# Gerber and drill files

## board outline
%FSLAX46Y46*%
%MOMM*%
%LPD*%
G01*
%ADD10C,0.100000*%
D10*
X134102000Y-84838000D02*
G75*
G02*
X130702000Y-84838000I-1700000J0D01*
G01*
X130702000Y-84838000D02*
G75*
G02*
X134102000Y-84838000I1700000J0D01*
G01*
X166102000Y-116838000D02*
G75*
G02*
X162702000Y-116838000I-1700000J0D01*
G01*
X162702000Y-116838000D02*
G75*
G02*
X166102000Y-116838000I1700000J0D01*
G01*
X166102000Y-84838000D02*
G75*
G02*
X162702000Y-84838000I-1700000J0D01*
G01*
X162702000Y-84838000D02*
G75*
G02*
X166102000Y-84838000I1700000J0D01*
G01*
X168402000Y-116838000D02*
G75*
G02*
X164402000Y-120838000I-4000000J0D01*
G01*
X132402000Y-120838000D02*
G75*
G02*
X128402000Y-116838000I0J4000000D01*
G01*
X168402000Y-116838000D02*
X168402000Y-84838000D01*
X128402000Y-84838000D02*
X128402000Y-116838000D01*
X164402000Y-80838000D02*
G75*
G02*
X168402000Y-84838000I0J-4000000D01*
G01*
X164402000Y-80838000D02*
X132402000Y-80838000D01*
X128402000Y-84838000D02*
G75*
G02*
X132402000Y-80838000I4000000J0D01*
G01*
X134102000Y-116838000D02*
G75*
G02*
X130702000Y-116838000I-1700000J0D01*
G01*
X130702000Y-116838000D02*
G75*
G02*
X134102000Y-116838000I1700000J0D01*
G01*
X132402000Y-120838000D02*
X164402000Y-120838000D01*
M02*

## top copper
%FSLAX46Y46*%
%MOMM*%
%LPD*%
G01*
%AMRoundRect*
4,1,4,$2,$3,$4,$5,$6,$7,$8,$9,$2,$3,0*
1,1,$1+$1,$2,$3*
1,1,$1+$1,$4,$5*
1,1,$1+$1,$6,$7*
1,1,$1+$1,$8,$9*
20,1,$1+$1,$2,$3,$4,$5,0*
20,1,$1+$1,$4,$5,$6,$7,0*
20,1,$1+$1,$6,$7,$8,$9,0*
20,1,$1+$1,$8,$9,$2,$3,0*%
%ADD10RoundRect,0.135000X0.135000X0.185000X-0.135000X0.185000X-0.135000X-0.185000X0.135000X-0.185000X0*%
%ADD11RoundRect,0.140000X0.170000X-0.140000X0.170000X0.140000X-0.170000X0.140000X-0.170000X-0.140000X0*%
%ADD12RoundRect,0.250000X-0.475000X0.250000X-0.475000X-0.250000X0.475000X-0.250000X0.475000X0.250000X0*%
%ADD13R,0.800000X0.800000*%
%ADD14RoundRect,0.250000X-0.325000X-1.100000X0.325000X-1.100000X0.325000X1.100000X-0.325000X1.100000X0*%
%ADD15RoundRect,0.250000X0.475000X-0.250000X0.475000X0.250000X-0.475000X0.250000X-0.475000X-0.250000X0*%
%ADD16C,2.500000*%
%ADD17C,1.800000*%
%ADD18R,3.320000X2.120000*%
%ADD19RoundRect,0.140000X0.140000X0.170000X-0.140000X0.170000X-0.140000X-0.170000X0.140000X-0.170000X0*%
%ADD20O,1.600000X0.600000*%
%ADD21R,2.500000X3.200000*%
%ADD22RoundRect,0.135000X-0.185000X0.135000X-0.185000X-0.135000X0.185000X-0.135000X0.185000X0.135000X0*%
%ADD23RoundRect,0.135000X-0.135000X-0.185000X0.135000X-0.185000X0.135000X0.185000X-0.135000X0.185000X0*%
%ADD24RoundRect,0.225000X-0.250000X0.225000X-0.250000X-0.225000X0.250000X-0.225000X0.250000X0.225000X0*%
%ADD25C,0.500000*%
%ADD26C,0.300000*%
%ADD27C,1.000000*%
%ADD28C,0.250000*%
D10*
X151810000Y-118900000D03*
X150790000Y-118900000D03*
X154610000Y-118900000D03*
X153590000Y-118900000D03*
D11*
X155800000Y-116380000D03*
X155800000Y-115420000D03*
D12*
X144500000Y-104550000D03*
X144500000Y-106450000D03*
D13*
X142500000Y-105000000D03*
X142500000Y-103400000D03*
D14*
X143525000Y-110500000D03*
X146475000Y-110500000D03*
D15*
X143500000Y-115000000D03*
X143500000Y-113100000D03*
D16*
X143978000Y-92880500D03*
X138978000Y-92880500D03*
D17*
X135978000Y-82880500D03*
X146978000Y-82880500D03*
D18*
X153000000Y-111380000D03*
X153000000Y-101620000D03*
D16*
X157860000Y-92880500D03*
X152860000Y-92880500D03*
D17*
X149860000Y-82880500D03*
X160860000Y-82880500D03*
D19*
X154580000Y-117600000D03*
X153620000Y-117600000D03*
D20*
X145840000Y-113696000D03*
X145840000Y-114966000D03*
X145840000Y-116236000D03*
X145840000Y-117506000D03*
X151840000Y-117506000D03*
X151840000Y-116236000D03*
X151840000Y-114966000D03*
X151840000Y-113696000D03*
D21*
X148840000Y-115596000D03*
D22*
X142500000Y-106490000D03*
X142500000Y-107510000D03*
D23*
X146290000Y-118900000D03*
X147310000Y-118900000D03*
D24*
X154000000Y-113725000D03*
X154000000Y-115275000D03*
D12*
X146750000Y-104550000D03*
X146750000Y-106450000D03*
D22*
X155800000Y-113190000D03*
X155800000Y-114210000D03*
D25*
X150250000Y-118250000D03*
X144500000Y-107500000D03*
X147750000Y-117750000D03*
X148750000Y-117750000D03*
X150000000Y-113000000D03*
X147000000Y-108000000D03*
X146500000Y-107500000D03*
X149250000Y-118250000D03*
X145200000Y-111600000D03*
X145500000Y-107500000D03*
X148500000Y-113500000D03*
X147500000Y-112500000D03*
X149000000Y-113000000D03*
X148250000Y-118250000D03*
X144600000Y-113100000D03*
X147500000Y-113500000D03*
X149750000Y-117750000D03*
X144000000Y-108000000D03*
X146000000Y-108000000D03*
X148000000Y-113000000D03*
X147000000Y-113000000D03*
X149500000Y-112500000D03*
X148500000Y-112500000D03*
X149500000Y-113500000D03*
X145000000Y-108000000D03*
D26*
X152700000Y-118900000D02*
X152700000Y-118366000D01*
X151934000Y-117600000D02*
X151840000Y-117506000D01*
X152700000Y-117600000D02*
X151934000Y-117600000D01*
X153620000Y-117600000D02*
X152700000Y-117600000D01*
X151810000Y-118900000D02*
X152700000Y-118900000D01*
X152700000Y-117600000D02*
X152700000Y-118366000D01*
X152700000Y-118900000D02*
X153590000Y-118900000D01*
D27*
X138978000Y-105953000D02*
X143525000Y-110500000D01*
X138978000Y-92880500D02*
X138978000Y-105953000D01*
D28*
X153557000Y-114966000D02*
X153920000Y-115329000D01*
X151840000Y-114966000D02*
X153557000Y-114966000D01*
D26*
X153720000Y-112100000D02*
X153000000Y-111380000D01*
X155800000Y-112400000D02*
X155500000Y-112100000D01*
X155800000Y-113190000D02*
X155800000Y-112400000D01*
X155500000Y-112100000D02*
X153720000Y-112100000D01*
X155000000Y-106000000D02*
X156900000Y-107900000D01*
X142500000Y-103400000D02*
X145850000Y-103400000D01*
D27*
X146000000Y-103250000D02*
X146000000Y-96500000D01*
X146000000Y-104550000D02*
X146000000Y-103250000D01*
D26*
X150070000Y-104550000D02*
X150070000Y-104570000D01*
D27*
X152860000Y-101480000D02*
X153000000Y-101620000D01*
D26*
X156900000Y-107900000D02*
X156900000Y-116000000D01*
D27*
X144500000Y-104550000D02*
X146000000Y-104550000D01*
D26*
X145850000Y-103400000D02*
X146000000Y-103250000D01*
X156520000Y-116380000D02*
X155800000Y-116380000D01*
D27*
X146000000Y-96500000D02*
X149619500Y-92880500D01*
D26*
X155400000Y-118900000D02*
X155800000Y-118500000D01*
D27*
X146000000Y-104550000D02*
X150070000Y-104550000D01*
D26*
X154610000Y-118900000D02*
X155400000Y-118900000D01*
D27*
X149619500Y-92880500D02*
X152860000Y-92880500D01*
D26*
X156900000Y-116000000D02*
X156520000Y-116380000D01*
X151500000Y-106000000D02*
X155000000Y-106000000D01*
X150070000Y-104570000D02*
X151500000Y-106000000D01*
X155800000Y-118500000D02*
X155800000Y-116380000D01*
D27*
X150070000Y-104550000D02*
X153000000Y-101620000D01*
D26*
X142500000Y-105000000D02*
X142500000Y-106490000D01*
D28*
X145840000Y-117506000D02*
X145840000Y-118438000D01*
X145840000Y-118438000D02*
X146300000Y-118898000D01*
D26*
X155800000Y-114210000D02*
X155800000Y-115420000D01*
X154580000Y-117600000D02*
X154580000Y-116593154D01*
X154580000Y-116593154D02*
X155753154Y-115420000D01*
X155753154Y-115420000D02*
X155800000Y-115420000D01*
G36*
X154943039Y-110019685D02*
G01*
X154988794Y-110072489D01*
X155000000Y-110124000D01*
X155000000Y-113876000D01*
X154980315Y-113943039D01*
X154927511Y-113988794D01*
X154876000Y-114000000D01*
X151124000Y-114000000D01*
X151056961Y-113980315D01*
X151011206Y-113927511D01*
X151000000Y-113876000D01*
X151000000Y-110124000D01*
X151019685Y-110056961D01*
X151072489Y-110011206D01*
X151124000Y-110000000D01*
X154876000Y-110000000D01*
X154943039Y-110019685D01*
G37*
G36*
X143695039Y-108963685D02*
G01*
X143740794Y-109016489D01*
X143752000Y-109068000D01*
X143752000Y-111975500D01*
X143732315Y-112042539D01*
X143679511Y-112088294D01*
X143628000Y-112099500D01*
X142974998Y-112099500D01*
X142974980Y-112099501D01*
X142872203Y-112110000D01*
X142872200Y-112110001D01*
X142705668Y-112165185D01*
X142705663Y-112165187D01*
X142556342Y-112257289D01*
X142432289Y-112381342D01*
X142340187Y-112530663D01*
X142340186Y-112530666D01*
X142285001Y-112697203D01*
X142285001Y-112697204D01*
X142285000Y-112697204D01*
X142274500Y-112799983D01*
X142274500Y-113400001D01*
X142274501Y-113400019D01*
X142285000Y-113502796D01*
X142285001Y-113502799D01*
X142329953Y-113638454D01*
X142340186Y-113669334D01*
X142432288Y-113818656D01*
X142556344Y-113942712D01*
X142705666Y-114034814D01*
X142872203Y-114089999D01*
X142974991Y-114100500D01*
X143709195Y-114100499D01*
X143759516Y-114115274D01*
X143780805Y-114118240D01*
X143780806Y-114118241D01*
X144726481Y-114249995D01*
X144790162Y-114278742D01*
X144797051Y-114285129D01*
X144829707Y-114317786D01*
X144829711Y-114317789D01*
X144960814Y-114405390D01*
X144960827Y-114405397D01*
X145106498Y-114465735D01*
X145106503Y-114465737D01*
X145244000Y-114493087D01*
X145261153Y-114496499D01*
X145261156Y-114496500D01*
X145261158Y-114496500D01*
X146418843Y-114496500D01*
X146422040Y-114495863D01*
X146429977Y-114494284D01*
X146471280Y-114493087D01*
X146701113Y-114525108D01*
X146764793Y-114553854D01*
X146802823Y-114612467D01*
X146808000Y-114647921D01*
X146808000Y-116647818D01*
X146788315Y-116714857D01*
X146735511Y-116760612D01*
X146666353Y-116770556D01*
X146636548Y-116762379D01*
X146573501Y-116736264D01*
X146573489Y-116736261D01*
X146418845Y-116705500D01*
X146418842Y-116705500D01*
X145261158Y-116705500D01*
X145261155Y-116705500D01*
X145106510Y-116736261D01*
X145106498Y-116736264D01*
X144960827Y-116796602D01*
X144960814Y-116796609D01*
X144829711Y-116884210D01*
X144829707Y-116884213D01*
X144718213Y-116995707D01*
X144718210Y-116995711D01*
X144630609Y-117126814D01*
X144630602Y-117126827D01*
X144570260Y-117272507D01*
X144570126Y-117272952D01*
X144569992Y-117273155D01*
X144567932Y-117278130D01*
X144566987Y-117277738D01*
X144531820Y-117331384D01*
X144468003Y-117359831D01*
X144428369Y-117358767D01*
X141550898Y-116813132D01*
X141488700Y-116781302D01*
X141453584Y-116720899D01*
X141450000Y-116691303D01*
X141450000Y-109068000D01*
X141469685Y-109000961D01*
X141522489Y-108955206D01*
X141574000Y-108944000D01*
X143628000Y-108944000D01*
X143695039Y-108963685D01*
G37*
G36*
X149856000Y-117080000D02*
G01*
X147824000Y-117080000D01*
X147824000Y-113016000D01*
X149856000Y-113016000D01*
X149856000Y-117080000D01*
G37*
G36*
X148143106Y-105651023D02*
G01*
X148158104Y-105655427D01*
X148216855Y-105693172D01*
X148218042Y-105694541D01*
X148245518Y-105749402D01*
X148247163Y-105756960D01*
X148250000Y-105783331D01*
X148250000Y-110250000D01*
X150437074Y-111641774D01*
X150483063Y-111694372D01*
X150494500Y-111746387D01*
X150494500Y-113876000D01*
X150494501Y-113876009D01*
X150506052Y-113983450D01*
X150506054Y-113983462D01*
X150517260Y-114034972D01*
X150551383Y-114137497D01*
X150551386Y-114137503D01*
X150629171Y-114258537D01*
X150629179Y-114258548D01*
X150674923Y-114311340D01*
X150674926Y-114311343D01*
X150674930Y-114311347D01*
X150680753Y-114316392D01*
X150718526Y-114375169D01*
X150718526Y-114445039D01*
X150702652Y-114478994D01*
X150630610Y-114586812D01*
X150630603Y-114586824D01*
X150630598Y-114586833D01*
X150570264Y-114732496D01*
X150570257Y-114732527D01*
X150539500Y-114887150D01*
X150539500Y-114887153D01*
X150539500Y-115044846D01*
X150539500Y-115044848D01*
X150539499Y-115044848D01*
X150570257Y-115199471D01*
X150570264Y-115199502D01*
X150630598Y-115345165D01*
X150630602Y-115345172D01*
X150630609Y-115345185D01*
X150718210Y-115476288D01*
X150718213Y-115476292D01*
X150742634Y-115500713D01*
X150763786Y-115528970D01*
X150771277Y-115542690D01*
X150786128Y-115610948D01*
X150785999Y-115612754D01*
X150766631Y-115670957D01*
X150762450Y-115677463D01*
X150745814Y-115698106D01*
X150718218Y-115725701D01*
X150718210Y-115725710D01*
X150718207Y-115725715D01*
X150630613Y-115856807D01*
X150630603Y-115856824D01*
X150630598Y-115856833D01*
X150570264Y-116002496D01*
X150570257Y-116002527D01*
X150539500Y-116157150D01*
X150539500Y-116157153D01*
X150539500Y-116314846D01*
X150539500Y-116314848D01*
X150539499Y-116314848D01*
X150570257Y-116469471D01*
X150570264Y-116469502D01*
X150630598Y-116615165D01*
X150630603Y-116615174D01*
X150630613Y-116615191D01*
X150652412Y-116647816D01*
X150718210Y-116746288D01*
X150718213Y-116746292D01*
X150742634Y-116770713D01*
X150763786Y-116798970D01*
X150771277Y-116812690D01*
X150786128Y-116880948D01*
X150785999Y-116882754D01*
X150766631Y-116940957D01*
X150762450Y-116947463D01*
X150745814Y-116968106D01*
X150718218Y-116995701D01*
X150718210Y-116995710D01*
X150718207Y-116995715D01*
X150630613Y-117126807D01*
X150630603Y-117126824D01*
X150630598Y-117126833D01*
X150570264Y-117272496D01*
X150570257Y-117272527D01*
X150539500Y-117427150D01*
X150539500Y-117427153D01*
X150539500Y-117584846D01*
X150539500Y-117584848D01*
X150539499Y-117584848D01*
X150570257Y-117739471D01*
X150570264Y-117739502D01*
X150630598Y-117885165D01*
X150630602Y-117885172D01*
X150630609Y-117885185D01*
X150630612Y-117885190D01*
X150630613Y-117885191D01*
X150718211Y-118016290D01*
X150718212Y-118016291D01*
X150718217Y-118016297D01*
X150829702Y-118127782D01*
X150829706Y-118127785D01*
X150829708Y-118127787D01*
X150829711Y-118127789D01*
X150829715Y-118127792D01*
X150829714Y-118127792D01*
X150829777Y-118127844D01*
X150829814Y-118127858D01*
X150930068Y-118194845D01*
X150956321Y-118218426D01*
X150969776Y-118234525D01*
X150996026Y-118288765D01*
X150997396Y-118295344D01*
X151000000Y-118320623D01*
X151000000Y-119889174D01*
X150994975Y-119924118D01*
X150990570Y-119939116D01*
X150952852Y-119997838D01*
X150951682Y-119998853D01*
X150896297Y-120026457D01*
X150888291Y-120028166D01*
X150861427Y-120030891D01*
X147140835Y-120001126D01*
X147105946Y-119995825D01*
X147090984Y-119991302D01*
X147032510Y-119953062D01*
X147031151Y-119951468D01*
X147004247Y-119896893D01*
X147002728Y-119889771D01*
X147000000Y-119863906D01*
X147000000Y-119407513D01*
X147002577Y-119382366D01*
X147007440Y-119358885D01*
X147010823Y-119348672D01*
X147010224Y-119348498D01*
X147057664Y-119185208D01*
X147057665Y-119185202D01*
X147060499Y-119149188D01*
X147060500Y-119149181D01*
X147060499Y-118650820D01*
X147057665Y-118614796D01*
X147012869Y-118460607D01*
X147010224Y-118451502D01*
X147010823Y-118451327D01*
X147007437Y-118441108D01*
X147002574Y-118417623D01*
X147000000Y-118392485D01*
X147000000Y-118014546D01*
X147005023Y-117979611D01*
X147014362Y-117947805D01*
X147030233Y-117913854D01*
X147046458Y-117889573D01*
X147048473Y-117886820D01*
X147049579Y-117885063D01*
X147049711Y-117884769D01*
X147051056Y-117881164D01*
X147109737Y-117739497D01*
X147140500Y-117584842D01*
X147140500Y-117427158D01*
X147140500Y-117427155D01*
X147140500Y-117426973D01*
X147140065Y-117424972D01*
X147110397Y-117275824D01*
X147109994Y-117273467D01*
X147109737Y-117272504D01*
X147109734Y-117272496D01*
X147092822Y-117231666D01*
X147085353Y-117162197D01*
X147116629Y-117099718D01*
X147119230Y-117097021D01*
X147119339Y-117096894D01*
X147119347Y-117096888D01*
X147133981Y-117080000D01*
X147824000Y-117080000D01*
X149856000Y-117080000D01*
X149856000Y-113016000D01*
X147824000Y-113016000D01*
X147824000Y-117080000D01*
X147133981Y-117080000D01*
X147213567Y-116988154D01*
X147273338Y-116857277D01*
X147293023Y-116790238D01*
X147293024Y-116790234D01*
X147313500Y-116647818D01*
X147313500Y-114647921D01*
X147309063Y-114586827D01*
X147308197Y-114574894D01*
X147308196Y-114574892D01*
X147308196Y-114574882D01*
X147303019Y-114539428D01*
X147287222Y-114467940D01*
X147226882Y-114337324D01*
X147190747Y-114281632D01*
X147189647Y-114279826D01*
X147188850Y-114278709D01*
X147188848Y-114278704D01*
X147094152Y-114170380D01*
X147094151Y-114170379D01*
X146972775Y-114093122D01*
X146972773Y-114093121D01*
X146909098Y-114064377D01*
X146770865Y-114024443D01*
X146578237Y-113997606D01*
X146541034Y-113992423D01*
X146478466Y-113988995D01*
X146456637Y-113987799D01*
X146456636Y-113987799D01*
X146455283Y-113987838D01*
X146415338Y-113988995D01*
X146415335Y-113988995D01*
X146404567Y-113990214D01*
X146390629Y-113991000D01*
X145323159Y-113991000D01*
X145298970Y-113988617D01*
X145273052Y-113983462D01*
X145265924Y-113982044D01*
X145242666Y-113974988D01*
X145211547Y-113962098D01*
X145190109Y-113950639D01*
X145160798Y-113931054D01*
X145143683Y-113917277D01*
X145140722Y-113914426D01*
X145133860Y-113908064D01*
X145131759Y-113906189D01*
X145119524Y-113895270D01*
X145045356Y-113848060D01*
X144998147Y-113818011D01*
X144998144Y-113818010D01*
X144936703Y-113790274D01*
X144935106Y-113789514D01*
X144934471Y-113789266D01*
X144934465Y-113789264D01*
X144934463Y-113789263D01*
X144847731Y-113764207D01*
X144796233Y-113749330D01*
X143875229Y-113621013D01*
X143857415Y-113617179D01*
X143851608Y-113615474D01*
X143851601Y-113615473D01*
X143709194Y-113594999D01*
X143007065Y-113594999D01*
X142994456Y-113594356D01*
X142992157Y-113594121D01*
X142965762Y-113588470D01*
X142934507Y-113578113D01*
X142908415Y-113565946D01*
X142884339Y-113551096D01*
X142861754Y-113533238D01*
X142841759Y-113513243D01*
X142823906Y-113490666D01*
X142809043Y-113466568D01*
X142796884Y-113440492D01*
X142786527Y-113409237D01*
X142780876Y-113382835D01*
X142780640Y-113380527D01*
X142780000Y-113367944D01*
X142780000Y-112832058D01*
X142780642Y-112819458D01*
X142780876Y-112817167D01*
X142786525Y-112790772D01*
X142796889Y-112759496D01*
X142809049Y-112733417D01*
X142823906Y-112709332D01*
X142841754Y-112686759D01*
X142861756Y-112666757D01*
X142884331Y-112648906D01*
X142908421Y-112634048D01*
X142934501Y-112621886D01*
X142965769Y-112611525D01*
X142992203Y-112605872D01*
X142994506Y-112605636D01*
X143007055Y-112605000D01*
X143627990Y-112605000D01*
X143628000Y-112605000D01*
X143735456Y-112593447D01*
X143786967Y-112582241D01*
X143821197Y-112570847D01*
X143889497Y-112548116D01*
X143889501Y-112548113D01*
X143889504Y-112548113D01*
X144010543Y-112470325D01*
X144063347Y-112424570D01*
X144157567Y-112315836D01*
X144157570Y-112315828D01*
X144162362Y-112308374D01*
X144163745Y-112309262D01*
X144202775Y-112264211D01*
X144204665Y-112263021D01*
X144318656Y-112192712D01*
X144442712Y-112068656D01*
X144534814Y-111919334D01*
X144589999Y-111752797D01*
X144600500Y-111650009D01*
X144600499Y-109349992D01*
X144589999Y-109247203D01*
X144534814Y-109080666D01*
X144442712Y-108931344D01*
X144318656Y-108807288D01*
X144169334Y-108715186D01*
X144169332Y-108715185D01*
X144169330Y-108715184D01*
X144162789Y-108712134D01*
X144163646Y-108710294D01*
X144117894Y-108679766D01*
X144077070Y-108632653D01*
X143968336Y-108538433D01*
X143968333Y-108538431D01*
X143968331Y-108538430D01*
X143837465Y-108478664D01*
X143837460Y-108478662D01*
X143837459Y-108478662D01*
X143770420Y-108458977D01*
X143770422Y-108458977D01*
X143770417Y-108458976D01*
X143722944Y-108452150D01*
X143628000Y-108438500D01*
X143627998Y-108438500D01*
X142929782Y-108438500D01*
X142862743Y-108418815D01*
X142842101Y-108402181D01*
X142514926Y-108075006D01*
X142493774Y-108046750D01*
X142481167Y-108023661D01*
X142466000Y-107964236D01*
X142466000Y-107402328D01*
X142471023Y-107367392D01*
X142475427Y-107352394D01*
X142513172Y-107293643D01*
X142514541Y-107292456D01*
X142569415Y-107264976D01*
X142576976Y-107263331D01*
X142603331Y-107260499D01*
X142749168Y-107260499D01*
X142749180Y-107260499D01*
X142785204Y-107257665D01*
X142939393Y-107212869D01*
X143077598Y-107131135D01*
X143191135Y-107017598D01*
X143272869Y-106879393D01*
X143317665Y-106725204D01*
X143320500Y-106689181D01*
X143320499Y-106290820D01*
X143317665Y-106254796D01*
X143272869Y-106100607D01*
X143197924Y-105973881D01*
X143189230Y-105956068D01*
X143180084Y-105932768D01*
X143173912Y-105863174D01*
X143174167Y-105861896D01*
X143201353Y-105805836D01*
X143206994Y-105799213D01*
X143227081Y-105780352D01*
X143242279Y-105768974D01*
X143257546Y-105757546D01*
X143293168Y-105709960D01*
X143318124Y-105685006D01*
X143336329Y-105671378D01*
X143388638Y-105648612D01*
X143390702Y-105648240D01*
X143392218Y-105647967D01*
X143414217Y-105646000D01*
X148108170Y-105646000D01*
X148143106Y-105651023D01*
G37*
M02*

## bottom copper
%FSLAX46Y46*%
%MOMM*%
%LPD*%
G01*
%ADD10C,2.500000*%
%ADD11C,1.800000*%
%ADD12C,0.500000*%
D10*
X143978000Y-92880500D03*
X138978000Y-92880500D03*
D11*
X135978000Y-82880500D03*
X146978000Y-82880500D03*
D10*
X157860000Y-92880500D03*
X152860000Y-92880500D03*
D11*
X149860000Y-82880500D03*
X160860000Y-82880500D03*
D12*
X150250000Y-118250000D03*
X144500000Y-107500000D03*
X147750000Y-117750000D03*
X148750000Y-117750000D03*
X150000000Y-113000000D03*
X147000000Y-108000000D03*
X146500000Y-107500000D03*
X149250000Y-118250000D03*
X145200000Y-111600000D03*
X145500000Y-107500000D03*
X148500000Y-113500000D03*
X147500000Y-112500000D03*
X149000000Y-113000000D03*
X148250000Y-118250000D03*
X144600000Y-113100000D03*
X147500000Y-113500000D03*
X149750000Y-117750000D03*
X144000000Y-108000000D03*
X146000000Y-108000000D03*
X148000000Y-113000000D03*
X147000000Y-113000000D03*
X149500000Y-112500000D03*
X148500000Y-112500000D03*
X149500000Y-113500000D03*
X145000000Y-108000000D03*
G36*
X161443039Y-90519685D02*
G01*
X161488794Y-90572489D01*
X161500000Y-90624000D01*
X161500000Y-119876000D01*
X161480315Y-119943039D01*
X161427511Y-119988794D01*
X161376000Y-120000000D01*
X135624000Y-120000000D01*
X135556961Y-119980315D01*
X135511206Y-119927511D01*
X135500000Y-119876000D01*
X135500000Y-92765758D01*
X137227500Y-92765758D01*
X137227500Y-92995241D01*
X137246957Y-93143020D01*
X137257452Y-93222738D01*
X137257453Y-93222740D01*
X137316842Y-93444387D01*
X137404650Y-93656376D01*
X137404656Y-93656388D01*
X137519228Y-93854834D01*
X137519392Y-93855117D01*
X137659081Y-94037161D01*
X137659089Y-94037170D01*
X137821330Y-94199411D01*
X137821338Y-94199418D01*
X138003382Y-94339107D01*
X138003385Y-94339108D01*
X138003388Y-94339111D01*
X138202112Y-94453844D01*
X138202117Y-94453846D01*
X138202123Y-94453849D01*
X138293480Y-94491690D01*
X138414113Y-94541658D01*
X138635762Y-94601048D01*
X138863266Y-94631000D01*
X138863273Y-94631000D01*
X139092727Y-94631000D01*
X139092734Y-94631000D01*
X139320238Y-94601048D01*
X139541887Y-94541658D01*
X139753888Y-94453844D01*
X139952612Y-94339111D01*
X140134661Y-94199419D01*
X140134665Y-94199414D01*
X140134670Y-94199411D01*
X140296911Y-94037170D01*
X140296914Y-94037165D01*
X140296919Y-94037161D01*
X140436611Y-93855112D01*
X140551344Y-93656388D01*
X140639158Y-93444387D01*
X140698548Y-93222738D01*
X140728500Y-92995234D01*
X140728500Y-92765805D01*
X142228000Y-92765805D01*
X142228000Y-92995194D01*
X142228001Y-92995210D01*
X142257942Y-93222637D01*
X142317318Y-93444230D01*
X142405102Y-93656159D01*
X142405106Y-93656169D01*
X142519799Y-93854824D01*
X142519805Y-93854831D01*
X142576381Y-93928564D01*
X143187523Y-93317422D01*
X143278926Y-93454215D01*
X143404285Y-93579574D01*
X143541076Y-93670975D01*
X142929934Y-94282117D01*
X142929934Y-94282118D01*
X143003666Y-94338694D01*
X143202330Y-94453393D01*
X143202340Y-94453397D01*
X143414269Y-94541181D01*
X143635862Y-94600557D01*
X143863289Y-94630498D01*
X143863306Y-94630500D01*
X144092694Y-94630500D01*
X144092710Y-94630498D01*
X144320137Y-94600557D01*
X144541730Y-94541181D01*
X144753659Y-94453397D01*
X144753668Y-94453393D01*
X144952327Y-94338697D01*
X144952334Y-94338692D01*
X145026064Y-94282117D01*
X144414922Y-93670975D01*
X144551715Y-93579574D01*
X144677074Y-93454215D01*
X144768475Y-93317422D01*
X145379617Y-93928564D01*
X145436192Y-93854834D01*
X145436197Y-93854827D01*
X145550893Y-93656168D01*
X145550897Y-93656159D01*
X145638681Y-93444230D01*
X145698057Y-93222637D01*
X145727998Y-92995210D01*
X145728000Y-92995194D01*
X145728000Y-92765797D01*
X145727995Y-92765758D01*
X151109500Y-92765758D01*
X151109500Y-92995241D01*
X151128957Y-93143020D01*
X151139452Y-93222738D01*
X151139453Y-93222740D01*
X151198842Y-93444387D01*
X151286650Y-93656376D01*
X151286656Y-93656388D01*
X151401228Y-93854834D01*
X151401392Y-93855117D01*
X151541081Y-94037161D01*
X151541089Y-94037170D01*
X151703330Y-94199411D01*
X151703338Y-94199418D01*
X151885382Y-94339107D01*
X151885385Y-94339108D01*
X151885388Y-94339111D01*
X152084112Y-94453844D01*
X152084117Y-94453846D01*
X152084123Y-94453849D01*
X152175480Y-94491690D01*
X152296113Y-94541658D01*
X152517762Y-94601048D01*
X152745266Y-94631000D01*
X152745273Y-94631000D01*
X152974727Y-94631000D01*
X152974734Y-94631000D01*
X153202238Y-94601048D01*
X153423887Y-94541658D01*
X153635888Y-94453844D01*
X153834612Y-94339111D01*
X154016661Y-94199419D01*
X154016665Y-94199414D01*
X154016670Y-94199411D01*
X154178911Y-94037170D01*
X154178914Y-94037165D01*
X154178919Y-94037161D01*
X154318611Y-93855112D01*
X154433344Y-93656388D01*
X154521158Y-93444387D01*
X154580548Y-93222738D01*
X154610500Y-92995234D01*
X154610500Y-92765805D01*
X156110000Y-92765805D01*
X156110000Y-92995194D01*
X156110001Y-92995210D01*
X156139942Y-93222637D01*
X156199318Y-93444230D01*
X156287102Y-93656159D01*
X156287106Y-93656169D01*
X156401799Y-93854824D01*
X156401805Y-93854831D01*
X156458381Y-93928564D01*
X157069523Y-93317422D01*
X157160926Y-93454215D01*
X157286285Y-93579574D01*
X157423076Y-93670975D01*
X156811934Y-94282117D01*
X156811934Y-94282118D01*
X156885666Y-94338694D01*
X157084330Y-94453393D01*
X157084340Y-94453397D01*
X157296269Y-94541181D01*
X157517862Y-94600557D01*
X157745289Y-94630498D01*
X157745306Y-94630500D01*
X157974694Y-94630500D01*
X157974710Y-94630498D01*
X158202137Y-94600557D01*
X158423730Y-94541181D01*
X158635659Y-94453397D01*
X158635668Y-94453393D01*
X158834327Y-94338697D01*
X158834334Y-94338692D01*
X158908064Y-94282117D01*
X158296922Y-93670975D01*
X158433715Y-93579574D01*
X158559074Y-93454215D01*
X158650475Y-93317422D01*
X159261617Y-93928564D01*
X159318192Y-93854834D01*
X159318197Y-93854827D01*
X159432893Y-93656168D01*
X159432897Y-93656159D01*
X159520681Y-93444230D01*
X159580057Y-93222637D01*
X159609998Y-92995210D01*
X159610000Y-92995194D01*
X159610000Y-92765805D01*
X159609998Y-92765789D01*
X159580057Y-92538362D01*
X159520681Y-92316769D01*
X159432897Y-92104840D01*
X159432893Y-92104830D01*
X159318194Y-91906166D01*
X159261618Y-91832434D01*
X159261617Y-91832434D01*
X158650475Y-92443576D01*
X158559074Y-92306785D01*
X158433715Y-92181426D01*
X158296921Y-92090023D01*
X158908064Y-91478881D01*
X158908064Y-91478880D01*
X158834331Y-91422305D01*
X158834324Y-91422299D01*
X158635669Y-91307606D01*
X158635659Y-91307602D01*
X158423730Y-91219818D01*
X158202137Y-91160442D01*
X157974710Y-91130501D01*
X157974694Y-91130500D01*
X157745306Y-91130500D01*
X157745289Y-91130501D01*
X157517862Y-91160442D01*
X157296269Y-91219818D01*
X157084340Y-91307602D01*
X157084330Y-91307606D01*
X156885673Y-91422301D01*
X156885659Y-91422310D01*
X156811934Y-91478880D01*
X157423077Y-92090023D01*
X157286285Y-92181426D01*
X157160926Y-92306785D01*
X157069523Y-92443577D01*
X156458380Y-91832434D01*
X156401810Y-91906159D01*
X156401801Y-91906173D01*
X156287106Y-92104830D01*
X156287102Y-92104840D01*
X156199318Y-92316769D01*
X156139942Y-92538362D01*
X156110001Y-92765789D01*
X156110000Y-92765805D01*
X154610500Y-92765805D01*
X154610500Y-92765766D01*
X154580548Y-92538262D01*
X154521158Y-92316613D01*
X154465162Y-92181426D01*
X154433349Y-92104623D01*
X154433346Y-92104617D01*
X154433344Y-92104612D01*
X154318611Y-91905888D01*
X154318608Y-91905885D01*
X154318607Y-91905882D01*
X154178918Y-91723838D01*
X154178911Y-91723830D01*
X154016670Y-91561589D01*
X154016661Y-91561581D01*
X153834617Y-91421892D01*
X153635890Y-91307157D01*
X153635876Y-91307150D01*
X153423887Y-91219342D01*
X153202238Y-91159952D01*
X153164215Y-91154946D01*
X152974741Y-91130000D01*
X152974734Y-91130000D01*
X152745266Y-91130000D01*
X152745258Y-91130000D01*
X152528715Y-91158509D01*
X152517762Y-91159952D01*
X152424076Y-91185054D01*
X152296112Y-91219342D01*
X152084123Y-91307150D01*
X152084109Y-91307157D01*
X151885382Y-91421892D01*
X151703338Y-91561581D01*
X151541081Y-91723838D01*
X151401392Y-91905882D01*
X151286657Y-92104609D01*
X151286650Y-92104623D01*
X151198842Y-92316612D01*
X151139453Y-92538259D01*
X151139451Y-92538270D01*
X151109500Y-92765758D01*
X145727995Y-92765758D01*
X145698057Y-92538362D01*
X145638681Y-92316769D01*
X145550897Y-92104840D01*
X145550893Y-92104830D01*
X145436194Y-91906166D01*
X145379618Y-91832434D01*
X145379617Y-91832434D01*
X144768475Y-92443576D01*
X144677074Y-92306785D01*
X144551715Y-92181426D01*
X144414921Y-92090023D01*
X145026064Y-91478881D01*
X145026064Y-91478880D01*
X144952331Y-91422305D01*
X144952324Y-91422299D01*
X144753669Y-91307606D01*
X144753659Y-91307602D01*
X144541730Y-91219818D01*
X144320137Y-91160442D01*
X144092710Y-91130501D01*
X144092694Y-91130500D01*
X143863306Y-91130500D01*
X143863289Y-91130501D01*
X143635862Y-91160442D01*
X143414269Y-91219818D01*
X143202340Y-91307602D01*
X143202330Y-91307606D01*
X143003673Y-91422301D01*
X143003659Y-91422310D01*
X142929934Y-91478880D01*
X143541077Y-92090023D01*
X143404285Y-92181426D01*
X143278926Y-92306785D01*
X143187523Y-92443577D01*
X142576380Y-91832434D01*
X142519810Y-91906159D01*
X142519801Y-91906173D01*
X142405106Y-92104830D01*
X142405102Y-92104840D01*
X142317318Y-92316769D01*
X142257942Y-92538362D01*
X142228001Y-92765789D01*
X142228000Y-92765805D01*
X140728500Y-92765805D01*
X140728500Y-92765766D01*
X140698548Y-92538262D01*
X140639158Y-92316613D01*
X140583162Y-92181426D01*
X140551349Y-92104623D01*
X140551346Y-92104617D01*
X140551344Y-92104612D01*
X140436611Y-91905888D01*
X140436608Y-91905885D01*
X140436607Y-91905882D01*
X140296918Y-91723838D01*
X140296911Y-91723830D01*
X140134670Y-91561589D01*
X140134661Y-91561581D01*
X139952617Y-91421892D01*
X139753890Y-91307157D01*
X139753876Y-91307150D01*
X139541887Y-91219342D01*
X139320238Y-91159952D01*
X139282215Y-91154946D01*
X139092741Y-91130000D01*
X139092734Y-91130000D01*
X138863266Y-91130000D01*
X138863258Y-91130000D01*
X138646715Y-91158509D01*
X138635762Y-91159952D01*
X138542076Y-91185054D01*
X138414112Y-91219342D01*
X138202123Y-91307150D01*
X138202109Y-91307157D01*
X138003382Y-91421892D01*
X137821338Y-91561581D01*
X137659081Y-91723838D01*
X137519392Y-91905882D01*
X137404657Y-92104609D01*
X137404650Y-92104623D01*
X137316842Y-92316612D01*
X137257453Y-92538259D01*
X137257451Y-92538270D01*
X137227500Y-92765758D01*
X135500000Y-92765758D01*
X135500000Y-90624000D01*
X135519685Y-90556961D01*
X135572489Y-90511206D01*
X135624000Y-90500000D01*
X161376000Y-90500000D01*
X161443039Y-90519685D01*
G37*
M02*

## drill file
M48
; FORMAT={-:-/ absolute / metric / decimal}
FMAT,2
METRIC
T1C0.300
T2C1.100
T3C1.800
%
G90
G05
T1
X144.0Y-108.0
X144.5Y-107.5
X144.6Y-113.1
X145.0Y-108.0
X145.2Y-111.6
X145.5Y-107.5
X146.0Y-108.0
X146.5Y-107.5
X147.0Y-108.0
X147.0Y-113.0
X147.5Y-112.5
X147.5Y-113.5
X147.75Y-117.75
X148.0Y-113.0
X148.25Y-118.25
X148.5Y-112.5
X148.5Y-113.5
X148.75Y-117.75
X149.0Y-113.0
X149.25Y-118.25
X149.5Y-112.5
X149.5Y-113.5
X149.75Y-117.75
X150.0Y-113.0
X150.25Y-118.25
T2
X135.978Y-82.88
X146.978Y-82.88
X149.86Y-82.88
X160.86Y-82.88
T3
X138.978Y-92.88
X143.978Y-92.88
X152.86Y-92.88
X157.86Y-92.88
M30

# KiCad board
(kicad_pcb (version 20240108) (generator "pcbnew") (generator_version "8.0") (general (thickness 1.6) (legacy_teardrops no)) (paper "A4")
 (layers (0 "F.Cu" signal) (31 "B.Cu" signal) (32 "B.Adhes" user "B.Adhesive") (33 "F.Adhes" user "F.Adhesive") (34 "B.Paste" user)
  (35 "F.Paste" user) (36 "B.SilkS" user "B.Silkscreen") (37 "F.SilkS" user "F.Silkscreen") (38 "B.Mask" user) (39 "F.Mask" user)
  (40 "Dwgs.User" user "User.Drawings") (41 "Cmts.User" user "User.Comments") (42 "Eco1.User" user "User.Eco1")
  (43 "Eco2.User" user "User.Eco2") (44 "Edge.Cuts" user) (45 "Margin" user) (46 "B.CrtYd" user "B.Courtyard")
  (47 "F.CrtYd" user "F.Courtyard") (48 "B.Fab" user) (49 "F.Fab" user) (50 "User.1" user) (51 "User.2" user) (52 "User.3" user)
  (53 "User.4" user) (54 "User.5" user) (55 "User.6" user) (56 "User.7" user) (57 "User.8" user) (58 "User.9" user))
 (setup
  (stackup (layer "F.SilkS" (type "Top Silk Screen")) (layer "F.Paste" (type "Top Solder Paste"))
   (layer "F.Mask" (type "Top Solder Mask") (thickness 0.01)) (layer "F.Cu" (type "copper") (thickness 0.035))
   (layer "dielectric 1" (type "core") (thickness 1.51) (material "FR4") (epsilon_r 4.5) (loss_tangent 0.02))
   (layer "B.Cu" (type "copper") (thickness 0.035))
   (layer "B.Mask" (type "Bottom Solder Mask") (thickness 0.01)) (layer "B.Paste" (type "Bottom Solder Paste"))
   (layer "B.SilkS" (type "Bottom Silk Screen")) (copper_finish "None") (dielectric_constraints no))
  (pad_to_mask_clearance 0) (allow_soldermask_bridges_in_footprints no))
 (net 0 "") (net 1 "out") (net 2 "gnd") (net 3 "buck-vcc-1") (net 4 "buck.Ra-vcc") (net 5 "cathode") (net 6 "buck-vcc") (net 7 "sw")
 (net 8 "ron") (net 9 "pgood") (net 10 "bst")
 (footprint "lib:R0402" (layer "F.Cu") (at 151.3 118.9 180)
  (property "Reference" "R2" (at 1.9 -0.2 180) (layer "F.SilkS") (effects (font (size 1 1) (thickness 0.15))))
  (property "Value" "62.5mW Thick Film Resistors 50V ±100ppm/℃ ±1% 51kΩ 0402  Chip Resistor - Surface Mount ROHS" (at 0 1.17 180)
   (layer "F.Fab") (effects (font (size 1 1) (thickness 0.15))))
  (pad "1" smd roundrect (at -0.51 0 180) (size 0.54 0.64) (layers "F.Cu" "F.Paste" "F.Mask") (roundrect_rratio 0.25) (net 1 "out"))
  (pad "2" smd roundrect (at 0.51 0 180) (size 0.54 0.64) (layers "F.Cu" "F.Paste" "F.Mask") (roundrect_rratio 0.25) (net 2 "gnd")))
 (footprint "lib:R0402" (layer "F.Cu") (at 154.1 118.9 180)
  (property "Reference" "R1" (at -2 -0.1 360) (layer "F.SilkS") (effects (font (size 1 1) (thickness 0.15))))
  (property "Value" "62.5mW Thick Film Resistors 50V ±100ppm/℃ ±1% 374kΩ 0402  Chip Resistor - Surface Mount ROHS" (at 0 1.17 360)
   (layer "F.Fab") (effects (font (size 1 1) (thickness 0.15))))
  (pad "1" smd roundrect (at -0.51 0 180) (size 0.54 0.64) (layers "F.Cu" "F.Paste" "F.Mask") (roundrect_rratio 0.25) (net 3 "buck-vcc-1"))
  (pad "2" smd roundrect (at 0.51 0 180) (size 0.54 0.64) (layers "F.Cu" "F.Paste" "F.Mask") (roundrect_rratio 0.25) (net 1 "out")))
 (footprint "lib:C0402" (layer "F.Cu") (at 155.8 115.9 90)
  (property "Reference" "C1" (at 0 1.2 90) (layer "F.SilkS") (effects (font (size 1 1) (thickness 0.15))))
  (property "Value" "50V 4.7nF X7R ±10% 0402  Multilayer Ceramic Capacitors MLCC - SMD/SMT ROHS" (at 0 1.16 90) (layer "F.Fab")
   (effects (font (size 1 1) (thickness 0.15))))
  (pad "1" smd roundrect (at -0.48 0 90) (size 0.56 0.62) (layers "F.Cu" "F.Paste" "F.Mask") (roundrect_rratio 0.25) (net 3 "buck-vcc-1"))
  (pad "2" smd roundrect (at 0.48 0 90) (size 0.56 0.62) (layers "F.Cu" "F.Paste" "F.Mask") (roundrect_rratio 0.25) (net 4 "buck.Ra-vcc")))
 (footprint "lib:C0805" (layer "F.Cu") (at 144.5 105.5 -90)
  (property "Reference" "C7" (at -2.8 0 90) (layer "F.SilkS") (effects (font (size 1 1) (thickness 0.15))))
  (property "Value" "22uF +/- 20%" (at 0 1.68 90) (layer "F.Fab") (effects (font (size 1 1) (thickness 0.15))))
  (pad "1" smd roundrect (at -0.95 0 270) (size 1 1.45) (layers "F.Cu" "F.Paste" "F.Mask") (roundrect_rratio 0.25) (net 3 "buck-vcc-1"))
  (pad "2" smd roundrect (at 0.95 0 270) (size 1 1.45) (layers "F.Cu" "F.Paste" "F.Mask") (roundrect_rratio 0.25) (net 2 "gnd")))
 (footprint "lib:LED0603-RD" (layer "F.Cu") (at 142.5 104.2 90)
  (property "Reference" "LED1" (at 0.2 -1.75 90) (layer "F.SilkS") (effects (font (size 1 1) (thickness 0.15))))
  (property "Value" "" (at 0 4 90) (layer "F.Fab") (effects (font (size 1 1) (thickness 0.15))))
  (pad "1" smd rect (at -0.8 0 180) (size 0.8 0.8) (layers "F.Cu" "F.Paste" "F.Mask") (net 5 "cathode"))
  (pad "2" smd rect (at 0.8 0 180) (size 0.8 0.8) (layers "F.Cu" "F.Paste" "F.Mask") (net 3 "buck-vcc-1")))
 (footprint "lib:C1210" (layer "F.Cu") (at 145 110.5)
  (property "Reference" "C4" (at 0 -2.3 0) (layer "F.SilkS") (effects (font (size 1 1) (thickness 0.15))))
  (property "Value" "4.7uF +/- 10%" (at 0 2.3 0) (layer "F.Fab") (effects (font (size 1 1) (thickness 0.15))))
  (pad "1" smd roundrect (at -1.475 0) (size 1.15 2.7) (layers "F.Cu" "F.Paste" "F.Mask") (roundrect_rratio 0.217391) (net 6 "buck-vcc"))
  (pad "2" smd roundrect (at 1.475 0) (size 1.15 2.7) (layers "F.Cu" "F.Paste" "F.Mask") (roundrect_rratio 0.217391) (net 2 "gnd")))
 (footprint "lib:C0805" (layer "F.Cu") (at 143.5 114.05 90)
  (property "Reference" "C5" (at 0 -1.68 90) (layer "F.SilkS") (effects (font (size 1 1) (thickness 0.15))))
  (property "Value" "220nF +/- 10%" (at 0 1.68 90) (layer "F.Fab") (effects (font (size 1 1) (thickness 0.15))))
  (pad "1" smd roundrect (at -0.95 0 90) (size 1 1.45) (layers "F.Cu" "F.Paste" "F.Mask") (roundrect_rratio 0.25) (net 6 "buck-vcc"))
  (pad "2" smd roundrect (at 0.95 0 90) (size 1 1.45) (layers "F.Cu" "F.Paste" "F.Mask") (roundrect_rratio 0.25) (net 2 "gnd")))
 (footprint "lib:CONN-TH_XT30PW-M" (layer "F.Cu") (at 141.478 87.8805 180)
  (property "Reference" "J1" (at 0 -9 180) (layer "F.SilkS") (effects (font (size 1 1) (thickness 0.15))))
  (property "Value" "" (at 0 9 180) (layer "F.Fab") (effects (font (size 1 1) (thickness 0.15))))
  (pad "1" thru_hole circle (at -2.5 -5 180) (size 2.5 2.5) (drill 1.799996) (layers "*.Cu" "*.Mask") (remove_unused_layers no)
   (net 2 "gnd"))
  (pad "2" thru_hole circle (at 2.5 -5 180) (size 2.5 2.5) (drill 1.799996) (layers "*.Cu" "*.Mask") (remove_unused_layers no)
   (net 6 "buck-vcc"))
  (pad "3" thru_hole circle (at 5.5 5 180) (size 1.8 1.8) (drill 1.100023) (layers "*.Cu" "*.Mask") (remove_unused_layers no))
  (pad "4" thru_hole circle (at -5.5 5 180) (size 1.8 1.8) (drill 1.100023) (layers "*.Cu" "*.Mask") (remove_unused_layers no)))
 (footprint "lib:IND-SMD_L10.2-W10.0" (layer "F.Cu") (at 153 106.5 -90)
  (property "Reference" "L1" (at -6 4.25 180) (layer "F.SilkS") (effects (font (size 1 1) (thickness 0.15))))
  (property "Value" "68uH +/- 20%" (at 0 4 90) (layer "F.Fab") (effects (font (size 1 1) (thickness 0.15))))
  (pad "1" smd rect (at 4.88 0 270) (size 2.12 3.32) (layers "F.Cu" "F.Paste" "F.Mask") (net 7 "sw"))
  (pad "2" smd rect (at -4.88 0 270) (size 2.12 3.32) (layers "F.Cu" "F.Paste" "F.Mask") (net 3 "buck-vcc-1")))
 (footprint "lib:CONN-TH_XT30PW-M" (layer "F.Cu") (at 155.36 87.8805 180)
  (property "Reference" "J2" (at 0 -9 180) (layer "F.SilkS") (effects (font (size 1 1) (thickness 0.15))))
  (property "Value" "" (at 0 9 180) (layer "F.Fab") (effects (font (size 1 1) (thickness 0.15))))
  (pad "1" thru_hole circle (at -2.5 -5 180) (size 2.5 2.5) (drill 1.799996) (layers "*.Cu" "*.Mask") (remove_unused_layers no)
   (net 2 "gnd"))
  (pad "2" thru_hole circle (at 2.5 -5 180) (size 2.5 2.5) (drill 1.799996) (layers "*.Cu" "*.Mask") (remove_unused_layers no)
   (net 3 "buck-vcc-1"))
  (pad "3" thru_hole circle (at 5.5 5 180) (size 1.8 1.8) (drill 1.100023) (layers "*.Cu" "*.Mask") (remove_unused_layers no))
  (pad "4" thru_hole circle (at -5.5 5 180) (size 1.8 1.8) (drill 1.100023) (layers "*.Cu" "*.Mask") (remove_unused_layers no)))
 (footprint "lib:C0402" (layer "F.Cu") (at 154.1 117.6 180)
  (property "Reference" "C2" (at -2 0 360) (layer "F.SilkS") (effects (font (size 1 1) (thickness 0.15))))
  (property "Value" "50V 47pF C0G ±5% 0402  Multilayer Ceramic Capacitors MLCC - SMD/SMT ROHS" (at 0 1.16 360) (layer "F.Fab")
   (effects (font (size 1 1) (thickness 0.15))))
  (pad "1" smd roundrect (at -0.48 0 180) (size 0.56 0.62) (layers "F.Cu" "F.Paste" "F.Mask") (roundrect_rratio 0.25) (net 4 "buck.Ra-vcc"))
  (pad "2" smd roundrect (at 0.48 0 180) (size 0.56 0.62) (layers "F.Cu" "F.Paste" "F.Mask") (roundrect_rratio 0.25) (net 1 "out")))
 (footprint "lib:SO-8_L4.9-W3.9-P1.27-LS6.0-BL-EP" (layer "F.Cu") (at 148.84 115.596 -90)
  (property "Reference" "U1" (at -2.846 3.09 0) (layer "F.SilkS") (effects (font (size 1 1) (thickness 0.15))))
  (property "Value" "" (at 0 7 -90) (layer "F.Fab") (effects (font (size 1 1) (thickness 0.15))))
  (pad "1" smd oval (at -1.9 3 270) (size 0.6 1.6) (layers "F.Cu" "F.Paste" "F.Mask") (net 2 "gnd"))
  (pad "2" smd oval (at -0.63 3 270) (size 0.6 1.6) (layers "F.Cu" "F.Paste" "F.Mask") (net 6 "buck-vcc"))
  (pad "3" smd oval (at 0.64 3 270) (size 0.6 1.6) (layers "F.Cu" "F.Paste" "F.Mask") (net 6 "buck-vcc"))
  (pad "4" smd oval (at 1.91 3 270) (size 0.6 1.6) (layers "F.Cu" "F.Paste" "F.Mask") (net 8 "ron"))
  (pad "5" smd oval (at 1.91 -3 270) (size 0.6 1.6) (layers "F.Cu" "F.Paste" "F.Mask") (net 1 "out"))
  (pad "6" smd oval (at 0.64 -3 270) (size 0.6 1.6) (layers "F.Cu" "F.Paste" "F.Mask") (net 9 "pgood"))
  (pad "7" smd oval (at -0.63 -3 270) (size 0.6 1.6) (layers "F.Cu" "F.Paste" "F.Mask") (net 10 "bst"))
  (pad "8" smd oval (at -1.9 -3 270) (size 0.6 1.6) (layers "F.Cu" "F.Paste" "F.Mask") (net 7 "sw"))
  (pad "9" smd rect (at 0 0 270) (size 3.2 2.5) (layers "F.Cu" "F.Paste" "F.Mask") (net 2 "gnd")))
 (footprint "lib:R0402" (layer "F.Cu") (at 142.5 107 -90)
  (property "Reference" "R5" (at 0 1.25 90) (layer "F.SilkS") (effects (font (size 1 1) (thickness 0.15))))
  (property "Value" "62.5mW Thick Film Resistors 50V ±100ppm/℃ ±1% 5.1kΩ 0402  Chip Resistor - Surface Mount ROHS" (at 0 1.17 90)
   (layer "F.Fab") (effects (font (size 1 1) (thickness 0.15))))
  (pad "1" smd roundrect (at -0.51 0 270) (size 0.54 0.64) (layers "F.Cu" "F.Paste" "F.Mask") (roundrect_rratio 0.25) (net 5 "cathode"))
  (pad "2" smd roundrect (at 0.51 0 270) (size 0.54 0.64) (layers "F.Cu" "F.Paste" "F.Mask") (roundrect_rratio 0.25) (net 2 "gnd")))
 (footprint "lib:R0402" (layer "F.Cu") (at 146.8 118.9)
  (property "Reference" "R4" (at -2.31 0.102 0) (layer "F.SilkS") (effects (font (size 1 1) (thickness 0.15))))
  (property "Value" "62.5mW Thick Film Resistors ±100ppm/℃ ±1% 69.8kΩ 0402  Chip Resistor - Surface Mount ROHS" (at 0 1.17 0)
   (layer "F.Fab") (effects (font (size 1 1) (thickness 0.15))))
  (pad "1" smd roundrect (at -0.51 0) (size 0.54 0.64) (layers "F.Cu" "F.Paste" "F.Mask") (roundrect_rratio 0.25) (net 8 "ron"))
  (pad "2" smd roundrect (at 0.51 0) (size 0.54 0.64) (layers "F.Cu" "F.Paste" "F.Mask") (roundrect_rratio 0.25) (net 2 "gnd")))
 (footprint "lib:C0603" (layer "F.Cu") (at 154 114.5 -90)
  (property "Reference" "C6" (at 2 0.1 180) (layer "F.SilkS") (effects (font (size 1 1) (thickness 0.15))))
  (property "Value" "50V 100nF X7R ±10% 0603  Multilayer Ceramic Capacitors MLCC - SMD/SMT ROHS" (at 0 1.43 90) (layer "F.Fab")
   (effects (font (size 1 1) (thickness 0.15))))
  (pad "1" smd roundrect (at -0.775 0 270) (size 0.9 0.95) (layers "F.Cu" "F.Paste" "F.Mask") (roundrect_rratio 0.25) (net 7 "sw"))
  (pad "2" smd roundrect (at 0.775 0 270) (size 0.9 0.95) (layers "F.Cu" "F.Paste" "F.Mask") (roundrect_rratio 0.25) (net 10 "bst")))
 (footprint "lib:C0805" (layer "F.Cu") (at 146.75 105.5 -90)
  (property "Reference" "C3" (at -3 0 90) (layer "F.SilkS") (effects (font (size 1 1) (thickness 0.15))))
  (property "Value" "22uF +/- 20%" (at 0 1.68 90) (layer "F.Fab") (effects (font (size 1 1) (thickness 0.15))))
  (pad "1" smd roundrect (at -0.95 0 270) (size 1 1.45) (layers "F.Cu" "F.Paste" "F.Mask") (roundrect_rratio 0.25) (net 3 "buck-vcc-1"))
  (pad "2" smd roundrect (at 0.95 0 270) (size 1 1.45) (layers "F.Cu" "F.Paste" "F.Mask") (roundrect_rratio 0.25) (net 2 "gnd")))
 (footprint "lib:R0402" (layer "F.Cu") (at 155.8 113.7 -90)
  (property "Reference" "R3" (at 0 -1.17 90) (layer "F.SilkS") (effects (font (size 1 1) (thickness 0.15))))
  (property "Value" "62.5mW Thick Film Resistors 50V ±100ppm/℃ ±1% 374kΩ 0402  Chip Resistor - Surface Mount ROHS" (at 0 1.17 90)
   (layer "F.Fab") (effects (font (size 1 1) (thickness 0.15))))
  (pad "1" smd roundrect (at -0.51 0 270) (size 0.54 0.64) (layers "F.Cu" "F.Paste" "F.Mask") (roundrect_rratio 0.25) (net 7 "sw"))
  (pad "2" smd roundrect (at 0.51 0 270) (size 0.54 0.64) (layers "F.Cu" "F.Paste" "F.Mask") (roundrect_rratio 0.25) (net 4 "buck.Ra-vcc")))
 (gr_circle (center 132.402 84.838) (end 134.102 84.838) (stroke (width 0.1) (type solid)) (fill none) (layer "Edge.Cuts"))
 (gr_circle (center 164.402 116.838) (end 166.102 116.838) (stroke (width 0.1) (type solid)) (fill none) (layer "Edge.Cuts"))
 (gr_circle (center 164.402 84.838) (end 166.102 84.838) (stroke (width 0.1) (type solid)) (fill none) (layer "Edge.Cuts"))
 (gr_arc (start 168.402 116.838) (mid 167.230427 119.666427) (end 164.402 120.838) (stroke (width 0.1) (type solid)) (layer "Edge.Cuts"))
 (gr_arc (start 132.402 120.838) (mid 129.573573 119.666427) (end 128.402 116.838) (stroke (width 0.1) (type solid)) (layer "Edge.Cuts"))
 (gr_line (start 168.402 116.838) (end 168.402 84.838) (stroke (width 0.1) (type solid)) (layer "Edge.Cuts"))
 (gr_line (start 128.402 84.838) (end 128.402 116.838) (stroke (width 0.1) (type solid)) (layer "Edge.Cuts"))
 (gr_arc (start 164.402 80.838) (mid 167.230427 82.009573) (end 168.402 84.838) (stroke (width 0.1) (type solid)) (layer "Edge.Cuts"))
 (gr_line (start 164.402 80.838) (end 132.402 80.838) (stroke (width 0.1) (type solid)) (layer "Edge.Cuts"))
 (gr_arc (start 128.402 84.838) (mid 129.573573 82.009573) (end 132.402 80.838) (stroke (width 0.1) (type solid)) (layer "Edge.Cuts"))
 (gr_circle (center 132.402 116.838) (end 134.102 116.838) (stroke (width 0.1) (type solid)) (fill none) (layer "Edge.Cuts"))
 (gr_line (start 132.402 120.838) (end 164.402 120.838) (stroke (width 0.1) (type solid)) (layer "Edge.Cuts"))
 (segment (start 152.7 118.9) (end 152.7 118.366) (width 0.3) (layer "F.Cu") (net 1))
 (segment (start 151.934 117.6) (end 151.84 117.506) (width 0.3) (layer "F.Cu") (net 1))
 (segment (start 152.7 117.6) (end 151.934 117.6) (width 0.3) (layer "F.Cu") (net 1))
 (segment (start 153.62 117.6) (end 152.7 117.6) (width 0.3) (layer "F.Cu") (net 1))
 (segment (start 151.81 118.9) (end 152.7 118.9) (width 0.3) (layer "F.Cu") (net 1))
 (segment (start 152.7 117.6) (end 152.7 118.366) (width 0.3) (layer "F.Cu") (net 1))
 (segment (start 152.7 118.9) (end 153.59 118.9) (width 0.3) (layer "F.Cu") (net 1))
 (segment (start 138.978 105.953) (end 143.525 110.5) (width 1) (layer "F.Cu") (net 6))
 (segment (start 138.978 92.8805) (end 138.978 105.953) (width 1) (layer "F.Cu") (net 6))
 (segment (start 153.557 114.966) (end 153.92 115.329) (width 0.25) (layer "F.Cu") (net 10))
 (segment (start 151.84 114.966) (end 153.557 114.966) (width 0.25) (layer "F.Cu") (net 10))
 (via (at 150.25 118.25) (size 0.5) (drill 0.3) (layers "F.Cu" "B.Cu") (free yes) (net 2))
 (via (at 144.5 107.5) (size 0.5) (drill 0.3) (layers "F.Cu" "B.Cu") (free yes) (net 2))
 (via (at 147.75 117.75) (size 0.5) (drill 0.3) (layers "F.Cu" "B.Cu") (free yes) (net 2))
 (via (at 148.75 117.75) (size 0.5) (drill 0.3) (layers "F.Cu" "B.Cu") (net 2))
 (via (at 150 113) (size 0.5) (drill 0.3) (layers "F.Cu" "B.Cu") (free yes) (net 2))
 (via (at 147 108) (size 0.5) (drill 0.3) (layers "F.Cu" "B.Cu") (free yes) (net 2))
 (via (at 146.5 107.5) (size 0.5) (drill 0.3) (layers "F.Cu" "B.Cu") (free yes) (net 2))
 (via (at 149.25 118.25) (size 0.5) (drill 0.3) (layers "F.Cu" "B.Cu") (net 2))
 (via (at 145.2 111.6) (size 0.5) (drill 0.3) (layers "F.Cu" "B.Cu") (free yes) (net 2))
 (via (at 145.5 107.5) (size 0.5) (drill 0.3) (layers "F.Cu" "B.Cu") (free yes) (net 2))
 (via (at 148.5 113.5) (size 0.5) (drill 0.3) (layers "F.Cu" "B.Cu") (free yes) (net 2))
 (via (at 147.5 112.5) (size 0.5) (drill 0.3) (layers "F.Cu" "B.Cu") (free yes) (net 2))
 (via (at 149 113) (size 0.5) (drill 0.3) (layers "F.Cu" "B.Cu") (free yes) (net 2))
 (via (at 148.25 118.25) (size 0.5) (drill 0.3) (layers "F.Cu" "B.Cu") (free yes) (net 2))
 (via (at 144.6 113.1) (size 0.5) (drill 0.3) (layers "F.Cu" "B.Cu") (free yes) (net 2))
 (via (at 147.5 113.5) (size 0.5) (drill 0.3) (layers "F.Cu" "B.Cu") (free yes) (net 2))
 (via (at 149.75 117.75) (size 0.5) (drill 0.3) (layers "F.Cu" "B.Cu") (free yes) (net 2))
 (via (at 144 108) (size 0.5) (drill 0.3) (layers "F.Cu" "B.Cu") (free yes) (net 2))
 (via (at 146 108) (size 0.5) (drill 0.3) (layers "F.Cu" "B.Cu") (free yes) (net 2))
 (via (at 148 113) (size 0.5) (drill 0.3) (layers "F.Cu" "B.Cu") (free yes) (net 2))
 (via (at 147 113) (size 0.5) (drill 0.3) (layers "F.Cu" "B.Cu") (free yes) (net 2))
 (via (at 149.5 112.5) (size 0.5) (drill 0.3) (layers "F.Cu" "B.Cu") (free yes) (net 2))
 (via (at 148.5 112.5) (size 0.5) (drill 0.3) (layers "F.Cu" "B.Cu") (free yes) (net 2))
 (via (at 149.5 113.5) (size 0.5) (drill 0.3) (layers "F.Cu" "B.Cu") (free yes) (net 2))
 (via (at 145 108) (size 0.5) (drill 0.3) (layers "F.Cu" "B.Cu") (free yes) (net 2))
 (segment (start 153.72 112.1) (end 153 111.38) (width 0.3) (layer "F.Cu") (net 7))
 (segment (start 155.8 112.4) (end 155.5 112.1) (width 0.3) (layer "F.Cu") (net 7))
 (segment (start 155.8 113.19) (end 155.8 112.4) (width 0.3) (layer "F.Cu") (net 7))
 (segment (start 155.5 112.1) (end 153.72 112.1) (width 0.3) (layer "F.Cu") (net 7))
 (segment (start 155 106) (end 156.9 107.9) (width 0.3) (layer "F.Cu") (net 3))
 (segment (start 142.5 103.4) (end 145.85 103.4) (width 0.3) (layer "F.Cu") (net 3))
 (segment (start 146 103.25) (end 146 96.5) (width 1) (layer "F.Cu") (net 3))
 (segment (start 146 104.55) (end 146 103.25) (width 1) (layer "F.Cu") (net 3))
 (segment (start 150.07 104.55) (end 150.07 104.57) (width 0.3) (layer "F.Cu") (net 3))
 (segment (start 152.86 101.48) (end 153 101.62) (width 1) (layer "F.Cu") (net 3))
 (segment (start 156.9 107.9) (end 156.9 116) (width 0.3) (layer "F.Cu") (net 3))
 (segment (start 144.5 104.55) (end 146 104.55) (width 1) (layer "F.Cu") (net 3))
 (segment (start 145.85 103.4) (end 146 103.25) (width 0.3) (layer "F.Cu") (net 3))
 (segment (start 156.52 116.38) (end 155.8 116.38) (width 0.3) (layer "F.Cu") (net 3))
 (segment (start 146 96.5) (end 149.6195 92.8805) (width 1) (layer "F.Cu") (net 3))
 (segment (start 155.4 118.9) (end 155.8 118.5) (width 0.3) (layer "F.Cu") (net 3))
 (segment (start 146 104.55) (end 150.07 104.55) (width 1) (layer "F.Cu") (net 3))
 (segment (start 154.61 118.9) (end 155.4 118.9) (width 0.3) (layer "F.Cu") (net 3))
 (segment (start 149.6195 92.8805) (end 152.86 92.8805) (width 1) (layer "F.Cu") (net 3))
 (segment (start 156.9 116) (end 156.52 116.38) (width 0.3) (layer "F.Cu") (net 3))
 (segment (start 151.5 106) (end 155 106) (width 0.3) (layer "F.Cu") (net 3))
 (segment (start 150.07 104.57) (end 151.5 106) (width 0.3) (layer "F.Cu") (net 3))
 (segment (start 155.8 118.5) (end 155.8 116.38) (width 0.3) (layer "F.Cu") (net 3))
 (segment (start 150.07 104.55) (end 153 101.62) (width 1) (layer "F.Cu") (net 3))
 (segment (start 142.5 105) (end 142.5 106.49) (width 0.3) (layer "F.Cu") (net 5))
 (segment (start 145.84 117.506) (end 145.84 118.438) (width 0.25) (layer "F.Cu") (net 8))
 (segment (start 145.84 118.438) (end 146.3 118.898) (width 0.25) (layer "F.Cu") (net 8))
 (segment (start 155.8 114.21) (end 155.8 115.42) (width 0.3) (layer "F.Cu") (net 4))
 (segment (start 154.58 117.6) (end 154.58 116.593154) (width 0.3) (layer "F.Cu") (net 4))
 (segment (start 154.58 116.593154) (end 155.753154 115.42) (width 0.3) (layer "F.Cu") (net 4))
 (segment (start 155.753154 115.42) (end 155.8 115.42) (width 0.3) (layer "F.Cu") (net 4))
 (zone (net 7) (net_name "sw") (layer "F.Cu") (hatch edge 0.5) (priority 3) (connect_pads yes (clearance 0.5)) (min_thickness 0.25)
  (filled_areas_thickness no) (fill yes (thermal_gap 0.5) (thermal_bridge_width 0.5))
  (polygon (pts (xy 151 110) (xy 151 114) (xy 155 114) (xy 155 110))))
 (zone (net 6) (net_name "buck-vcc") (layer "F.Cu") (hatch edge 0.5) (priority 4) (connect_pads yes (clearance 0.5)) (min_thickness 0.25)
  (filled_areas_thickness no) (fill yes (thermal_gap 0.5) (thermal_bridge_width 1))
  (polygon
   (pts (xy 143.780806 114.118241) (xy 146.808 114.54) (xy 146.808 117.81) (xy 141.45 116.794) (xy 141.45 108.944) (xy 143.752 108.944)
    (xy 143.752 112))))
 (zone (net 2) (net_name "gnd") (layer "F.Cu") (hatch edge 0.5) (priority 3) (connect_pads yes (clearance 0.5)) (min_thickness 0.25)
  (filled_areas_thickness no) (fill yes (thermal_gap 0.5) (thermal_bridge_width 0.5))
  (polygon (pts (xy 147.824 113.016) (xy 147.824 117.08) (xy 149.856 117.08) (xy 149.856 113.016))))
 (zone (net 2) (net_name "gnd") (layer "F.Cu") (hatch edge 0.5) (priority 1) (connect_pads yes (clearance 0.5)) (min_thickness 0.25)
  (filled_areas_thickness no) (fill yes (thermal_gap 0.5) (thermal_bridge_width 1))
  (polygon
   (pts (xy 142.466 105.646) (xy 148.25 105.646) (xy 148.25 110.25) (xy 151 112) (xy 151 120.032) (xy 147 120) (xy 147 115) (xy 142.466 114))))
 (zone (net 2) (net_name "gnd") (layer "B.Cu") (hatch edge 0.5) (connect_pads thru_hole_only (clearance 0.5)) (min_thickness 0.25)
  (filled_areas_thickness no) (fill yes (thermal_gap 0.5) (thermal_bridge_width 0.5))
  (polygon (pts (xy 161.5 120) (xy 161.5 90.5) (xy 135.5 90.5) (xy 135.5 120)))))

